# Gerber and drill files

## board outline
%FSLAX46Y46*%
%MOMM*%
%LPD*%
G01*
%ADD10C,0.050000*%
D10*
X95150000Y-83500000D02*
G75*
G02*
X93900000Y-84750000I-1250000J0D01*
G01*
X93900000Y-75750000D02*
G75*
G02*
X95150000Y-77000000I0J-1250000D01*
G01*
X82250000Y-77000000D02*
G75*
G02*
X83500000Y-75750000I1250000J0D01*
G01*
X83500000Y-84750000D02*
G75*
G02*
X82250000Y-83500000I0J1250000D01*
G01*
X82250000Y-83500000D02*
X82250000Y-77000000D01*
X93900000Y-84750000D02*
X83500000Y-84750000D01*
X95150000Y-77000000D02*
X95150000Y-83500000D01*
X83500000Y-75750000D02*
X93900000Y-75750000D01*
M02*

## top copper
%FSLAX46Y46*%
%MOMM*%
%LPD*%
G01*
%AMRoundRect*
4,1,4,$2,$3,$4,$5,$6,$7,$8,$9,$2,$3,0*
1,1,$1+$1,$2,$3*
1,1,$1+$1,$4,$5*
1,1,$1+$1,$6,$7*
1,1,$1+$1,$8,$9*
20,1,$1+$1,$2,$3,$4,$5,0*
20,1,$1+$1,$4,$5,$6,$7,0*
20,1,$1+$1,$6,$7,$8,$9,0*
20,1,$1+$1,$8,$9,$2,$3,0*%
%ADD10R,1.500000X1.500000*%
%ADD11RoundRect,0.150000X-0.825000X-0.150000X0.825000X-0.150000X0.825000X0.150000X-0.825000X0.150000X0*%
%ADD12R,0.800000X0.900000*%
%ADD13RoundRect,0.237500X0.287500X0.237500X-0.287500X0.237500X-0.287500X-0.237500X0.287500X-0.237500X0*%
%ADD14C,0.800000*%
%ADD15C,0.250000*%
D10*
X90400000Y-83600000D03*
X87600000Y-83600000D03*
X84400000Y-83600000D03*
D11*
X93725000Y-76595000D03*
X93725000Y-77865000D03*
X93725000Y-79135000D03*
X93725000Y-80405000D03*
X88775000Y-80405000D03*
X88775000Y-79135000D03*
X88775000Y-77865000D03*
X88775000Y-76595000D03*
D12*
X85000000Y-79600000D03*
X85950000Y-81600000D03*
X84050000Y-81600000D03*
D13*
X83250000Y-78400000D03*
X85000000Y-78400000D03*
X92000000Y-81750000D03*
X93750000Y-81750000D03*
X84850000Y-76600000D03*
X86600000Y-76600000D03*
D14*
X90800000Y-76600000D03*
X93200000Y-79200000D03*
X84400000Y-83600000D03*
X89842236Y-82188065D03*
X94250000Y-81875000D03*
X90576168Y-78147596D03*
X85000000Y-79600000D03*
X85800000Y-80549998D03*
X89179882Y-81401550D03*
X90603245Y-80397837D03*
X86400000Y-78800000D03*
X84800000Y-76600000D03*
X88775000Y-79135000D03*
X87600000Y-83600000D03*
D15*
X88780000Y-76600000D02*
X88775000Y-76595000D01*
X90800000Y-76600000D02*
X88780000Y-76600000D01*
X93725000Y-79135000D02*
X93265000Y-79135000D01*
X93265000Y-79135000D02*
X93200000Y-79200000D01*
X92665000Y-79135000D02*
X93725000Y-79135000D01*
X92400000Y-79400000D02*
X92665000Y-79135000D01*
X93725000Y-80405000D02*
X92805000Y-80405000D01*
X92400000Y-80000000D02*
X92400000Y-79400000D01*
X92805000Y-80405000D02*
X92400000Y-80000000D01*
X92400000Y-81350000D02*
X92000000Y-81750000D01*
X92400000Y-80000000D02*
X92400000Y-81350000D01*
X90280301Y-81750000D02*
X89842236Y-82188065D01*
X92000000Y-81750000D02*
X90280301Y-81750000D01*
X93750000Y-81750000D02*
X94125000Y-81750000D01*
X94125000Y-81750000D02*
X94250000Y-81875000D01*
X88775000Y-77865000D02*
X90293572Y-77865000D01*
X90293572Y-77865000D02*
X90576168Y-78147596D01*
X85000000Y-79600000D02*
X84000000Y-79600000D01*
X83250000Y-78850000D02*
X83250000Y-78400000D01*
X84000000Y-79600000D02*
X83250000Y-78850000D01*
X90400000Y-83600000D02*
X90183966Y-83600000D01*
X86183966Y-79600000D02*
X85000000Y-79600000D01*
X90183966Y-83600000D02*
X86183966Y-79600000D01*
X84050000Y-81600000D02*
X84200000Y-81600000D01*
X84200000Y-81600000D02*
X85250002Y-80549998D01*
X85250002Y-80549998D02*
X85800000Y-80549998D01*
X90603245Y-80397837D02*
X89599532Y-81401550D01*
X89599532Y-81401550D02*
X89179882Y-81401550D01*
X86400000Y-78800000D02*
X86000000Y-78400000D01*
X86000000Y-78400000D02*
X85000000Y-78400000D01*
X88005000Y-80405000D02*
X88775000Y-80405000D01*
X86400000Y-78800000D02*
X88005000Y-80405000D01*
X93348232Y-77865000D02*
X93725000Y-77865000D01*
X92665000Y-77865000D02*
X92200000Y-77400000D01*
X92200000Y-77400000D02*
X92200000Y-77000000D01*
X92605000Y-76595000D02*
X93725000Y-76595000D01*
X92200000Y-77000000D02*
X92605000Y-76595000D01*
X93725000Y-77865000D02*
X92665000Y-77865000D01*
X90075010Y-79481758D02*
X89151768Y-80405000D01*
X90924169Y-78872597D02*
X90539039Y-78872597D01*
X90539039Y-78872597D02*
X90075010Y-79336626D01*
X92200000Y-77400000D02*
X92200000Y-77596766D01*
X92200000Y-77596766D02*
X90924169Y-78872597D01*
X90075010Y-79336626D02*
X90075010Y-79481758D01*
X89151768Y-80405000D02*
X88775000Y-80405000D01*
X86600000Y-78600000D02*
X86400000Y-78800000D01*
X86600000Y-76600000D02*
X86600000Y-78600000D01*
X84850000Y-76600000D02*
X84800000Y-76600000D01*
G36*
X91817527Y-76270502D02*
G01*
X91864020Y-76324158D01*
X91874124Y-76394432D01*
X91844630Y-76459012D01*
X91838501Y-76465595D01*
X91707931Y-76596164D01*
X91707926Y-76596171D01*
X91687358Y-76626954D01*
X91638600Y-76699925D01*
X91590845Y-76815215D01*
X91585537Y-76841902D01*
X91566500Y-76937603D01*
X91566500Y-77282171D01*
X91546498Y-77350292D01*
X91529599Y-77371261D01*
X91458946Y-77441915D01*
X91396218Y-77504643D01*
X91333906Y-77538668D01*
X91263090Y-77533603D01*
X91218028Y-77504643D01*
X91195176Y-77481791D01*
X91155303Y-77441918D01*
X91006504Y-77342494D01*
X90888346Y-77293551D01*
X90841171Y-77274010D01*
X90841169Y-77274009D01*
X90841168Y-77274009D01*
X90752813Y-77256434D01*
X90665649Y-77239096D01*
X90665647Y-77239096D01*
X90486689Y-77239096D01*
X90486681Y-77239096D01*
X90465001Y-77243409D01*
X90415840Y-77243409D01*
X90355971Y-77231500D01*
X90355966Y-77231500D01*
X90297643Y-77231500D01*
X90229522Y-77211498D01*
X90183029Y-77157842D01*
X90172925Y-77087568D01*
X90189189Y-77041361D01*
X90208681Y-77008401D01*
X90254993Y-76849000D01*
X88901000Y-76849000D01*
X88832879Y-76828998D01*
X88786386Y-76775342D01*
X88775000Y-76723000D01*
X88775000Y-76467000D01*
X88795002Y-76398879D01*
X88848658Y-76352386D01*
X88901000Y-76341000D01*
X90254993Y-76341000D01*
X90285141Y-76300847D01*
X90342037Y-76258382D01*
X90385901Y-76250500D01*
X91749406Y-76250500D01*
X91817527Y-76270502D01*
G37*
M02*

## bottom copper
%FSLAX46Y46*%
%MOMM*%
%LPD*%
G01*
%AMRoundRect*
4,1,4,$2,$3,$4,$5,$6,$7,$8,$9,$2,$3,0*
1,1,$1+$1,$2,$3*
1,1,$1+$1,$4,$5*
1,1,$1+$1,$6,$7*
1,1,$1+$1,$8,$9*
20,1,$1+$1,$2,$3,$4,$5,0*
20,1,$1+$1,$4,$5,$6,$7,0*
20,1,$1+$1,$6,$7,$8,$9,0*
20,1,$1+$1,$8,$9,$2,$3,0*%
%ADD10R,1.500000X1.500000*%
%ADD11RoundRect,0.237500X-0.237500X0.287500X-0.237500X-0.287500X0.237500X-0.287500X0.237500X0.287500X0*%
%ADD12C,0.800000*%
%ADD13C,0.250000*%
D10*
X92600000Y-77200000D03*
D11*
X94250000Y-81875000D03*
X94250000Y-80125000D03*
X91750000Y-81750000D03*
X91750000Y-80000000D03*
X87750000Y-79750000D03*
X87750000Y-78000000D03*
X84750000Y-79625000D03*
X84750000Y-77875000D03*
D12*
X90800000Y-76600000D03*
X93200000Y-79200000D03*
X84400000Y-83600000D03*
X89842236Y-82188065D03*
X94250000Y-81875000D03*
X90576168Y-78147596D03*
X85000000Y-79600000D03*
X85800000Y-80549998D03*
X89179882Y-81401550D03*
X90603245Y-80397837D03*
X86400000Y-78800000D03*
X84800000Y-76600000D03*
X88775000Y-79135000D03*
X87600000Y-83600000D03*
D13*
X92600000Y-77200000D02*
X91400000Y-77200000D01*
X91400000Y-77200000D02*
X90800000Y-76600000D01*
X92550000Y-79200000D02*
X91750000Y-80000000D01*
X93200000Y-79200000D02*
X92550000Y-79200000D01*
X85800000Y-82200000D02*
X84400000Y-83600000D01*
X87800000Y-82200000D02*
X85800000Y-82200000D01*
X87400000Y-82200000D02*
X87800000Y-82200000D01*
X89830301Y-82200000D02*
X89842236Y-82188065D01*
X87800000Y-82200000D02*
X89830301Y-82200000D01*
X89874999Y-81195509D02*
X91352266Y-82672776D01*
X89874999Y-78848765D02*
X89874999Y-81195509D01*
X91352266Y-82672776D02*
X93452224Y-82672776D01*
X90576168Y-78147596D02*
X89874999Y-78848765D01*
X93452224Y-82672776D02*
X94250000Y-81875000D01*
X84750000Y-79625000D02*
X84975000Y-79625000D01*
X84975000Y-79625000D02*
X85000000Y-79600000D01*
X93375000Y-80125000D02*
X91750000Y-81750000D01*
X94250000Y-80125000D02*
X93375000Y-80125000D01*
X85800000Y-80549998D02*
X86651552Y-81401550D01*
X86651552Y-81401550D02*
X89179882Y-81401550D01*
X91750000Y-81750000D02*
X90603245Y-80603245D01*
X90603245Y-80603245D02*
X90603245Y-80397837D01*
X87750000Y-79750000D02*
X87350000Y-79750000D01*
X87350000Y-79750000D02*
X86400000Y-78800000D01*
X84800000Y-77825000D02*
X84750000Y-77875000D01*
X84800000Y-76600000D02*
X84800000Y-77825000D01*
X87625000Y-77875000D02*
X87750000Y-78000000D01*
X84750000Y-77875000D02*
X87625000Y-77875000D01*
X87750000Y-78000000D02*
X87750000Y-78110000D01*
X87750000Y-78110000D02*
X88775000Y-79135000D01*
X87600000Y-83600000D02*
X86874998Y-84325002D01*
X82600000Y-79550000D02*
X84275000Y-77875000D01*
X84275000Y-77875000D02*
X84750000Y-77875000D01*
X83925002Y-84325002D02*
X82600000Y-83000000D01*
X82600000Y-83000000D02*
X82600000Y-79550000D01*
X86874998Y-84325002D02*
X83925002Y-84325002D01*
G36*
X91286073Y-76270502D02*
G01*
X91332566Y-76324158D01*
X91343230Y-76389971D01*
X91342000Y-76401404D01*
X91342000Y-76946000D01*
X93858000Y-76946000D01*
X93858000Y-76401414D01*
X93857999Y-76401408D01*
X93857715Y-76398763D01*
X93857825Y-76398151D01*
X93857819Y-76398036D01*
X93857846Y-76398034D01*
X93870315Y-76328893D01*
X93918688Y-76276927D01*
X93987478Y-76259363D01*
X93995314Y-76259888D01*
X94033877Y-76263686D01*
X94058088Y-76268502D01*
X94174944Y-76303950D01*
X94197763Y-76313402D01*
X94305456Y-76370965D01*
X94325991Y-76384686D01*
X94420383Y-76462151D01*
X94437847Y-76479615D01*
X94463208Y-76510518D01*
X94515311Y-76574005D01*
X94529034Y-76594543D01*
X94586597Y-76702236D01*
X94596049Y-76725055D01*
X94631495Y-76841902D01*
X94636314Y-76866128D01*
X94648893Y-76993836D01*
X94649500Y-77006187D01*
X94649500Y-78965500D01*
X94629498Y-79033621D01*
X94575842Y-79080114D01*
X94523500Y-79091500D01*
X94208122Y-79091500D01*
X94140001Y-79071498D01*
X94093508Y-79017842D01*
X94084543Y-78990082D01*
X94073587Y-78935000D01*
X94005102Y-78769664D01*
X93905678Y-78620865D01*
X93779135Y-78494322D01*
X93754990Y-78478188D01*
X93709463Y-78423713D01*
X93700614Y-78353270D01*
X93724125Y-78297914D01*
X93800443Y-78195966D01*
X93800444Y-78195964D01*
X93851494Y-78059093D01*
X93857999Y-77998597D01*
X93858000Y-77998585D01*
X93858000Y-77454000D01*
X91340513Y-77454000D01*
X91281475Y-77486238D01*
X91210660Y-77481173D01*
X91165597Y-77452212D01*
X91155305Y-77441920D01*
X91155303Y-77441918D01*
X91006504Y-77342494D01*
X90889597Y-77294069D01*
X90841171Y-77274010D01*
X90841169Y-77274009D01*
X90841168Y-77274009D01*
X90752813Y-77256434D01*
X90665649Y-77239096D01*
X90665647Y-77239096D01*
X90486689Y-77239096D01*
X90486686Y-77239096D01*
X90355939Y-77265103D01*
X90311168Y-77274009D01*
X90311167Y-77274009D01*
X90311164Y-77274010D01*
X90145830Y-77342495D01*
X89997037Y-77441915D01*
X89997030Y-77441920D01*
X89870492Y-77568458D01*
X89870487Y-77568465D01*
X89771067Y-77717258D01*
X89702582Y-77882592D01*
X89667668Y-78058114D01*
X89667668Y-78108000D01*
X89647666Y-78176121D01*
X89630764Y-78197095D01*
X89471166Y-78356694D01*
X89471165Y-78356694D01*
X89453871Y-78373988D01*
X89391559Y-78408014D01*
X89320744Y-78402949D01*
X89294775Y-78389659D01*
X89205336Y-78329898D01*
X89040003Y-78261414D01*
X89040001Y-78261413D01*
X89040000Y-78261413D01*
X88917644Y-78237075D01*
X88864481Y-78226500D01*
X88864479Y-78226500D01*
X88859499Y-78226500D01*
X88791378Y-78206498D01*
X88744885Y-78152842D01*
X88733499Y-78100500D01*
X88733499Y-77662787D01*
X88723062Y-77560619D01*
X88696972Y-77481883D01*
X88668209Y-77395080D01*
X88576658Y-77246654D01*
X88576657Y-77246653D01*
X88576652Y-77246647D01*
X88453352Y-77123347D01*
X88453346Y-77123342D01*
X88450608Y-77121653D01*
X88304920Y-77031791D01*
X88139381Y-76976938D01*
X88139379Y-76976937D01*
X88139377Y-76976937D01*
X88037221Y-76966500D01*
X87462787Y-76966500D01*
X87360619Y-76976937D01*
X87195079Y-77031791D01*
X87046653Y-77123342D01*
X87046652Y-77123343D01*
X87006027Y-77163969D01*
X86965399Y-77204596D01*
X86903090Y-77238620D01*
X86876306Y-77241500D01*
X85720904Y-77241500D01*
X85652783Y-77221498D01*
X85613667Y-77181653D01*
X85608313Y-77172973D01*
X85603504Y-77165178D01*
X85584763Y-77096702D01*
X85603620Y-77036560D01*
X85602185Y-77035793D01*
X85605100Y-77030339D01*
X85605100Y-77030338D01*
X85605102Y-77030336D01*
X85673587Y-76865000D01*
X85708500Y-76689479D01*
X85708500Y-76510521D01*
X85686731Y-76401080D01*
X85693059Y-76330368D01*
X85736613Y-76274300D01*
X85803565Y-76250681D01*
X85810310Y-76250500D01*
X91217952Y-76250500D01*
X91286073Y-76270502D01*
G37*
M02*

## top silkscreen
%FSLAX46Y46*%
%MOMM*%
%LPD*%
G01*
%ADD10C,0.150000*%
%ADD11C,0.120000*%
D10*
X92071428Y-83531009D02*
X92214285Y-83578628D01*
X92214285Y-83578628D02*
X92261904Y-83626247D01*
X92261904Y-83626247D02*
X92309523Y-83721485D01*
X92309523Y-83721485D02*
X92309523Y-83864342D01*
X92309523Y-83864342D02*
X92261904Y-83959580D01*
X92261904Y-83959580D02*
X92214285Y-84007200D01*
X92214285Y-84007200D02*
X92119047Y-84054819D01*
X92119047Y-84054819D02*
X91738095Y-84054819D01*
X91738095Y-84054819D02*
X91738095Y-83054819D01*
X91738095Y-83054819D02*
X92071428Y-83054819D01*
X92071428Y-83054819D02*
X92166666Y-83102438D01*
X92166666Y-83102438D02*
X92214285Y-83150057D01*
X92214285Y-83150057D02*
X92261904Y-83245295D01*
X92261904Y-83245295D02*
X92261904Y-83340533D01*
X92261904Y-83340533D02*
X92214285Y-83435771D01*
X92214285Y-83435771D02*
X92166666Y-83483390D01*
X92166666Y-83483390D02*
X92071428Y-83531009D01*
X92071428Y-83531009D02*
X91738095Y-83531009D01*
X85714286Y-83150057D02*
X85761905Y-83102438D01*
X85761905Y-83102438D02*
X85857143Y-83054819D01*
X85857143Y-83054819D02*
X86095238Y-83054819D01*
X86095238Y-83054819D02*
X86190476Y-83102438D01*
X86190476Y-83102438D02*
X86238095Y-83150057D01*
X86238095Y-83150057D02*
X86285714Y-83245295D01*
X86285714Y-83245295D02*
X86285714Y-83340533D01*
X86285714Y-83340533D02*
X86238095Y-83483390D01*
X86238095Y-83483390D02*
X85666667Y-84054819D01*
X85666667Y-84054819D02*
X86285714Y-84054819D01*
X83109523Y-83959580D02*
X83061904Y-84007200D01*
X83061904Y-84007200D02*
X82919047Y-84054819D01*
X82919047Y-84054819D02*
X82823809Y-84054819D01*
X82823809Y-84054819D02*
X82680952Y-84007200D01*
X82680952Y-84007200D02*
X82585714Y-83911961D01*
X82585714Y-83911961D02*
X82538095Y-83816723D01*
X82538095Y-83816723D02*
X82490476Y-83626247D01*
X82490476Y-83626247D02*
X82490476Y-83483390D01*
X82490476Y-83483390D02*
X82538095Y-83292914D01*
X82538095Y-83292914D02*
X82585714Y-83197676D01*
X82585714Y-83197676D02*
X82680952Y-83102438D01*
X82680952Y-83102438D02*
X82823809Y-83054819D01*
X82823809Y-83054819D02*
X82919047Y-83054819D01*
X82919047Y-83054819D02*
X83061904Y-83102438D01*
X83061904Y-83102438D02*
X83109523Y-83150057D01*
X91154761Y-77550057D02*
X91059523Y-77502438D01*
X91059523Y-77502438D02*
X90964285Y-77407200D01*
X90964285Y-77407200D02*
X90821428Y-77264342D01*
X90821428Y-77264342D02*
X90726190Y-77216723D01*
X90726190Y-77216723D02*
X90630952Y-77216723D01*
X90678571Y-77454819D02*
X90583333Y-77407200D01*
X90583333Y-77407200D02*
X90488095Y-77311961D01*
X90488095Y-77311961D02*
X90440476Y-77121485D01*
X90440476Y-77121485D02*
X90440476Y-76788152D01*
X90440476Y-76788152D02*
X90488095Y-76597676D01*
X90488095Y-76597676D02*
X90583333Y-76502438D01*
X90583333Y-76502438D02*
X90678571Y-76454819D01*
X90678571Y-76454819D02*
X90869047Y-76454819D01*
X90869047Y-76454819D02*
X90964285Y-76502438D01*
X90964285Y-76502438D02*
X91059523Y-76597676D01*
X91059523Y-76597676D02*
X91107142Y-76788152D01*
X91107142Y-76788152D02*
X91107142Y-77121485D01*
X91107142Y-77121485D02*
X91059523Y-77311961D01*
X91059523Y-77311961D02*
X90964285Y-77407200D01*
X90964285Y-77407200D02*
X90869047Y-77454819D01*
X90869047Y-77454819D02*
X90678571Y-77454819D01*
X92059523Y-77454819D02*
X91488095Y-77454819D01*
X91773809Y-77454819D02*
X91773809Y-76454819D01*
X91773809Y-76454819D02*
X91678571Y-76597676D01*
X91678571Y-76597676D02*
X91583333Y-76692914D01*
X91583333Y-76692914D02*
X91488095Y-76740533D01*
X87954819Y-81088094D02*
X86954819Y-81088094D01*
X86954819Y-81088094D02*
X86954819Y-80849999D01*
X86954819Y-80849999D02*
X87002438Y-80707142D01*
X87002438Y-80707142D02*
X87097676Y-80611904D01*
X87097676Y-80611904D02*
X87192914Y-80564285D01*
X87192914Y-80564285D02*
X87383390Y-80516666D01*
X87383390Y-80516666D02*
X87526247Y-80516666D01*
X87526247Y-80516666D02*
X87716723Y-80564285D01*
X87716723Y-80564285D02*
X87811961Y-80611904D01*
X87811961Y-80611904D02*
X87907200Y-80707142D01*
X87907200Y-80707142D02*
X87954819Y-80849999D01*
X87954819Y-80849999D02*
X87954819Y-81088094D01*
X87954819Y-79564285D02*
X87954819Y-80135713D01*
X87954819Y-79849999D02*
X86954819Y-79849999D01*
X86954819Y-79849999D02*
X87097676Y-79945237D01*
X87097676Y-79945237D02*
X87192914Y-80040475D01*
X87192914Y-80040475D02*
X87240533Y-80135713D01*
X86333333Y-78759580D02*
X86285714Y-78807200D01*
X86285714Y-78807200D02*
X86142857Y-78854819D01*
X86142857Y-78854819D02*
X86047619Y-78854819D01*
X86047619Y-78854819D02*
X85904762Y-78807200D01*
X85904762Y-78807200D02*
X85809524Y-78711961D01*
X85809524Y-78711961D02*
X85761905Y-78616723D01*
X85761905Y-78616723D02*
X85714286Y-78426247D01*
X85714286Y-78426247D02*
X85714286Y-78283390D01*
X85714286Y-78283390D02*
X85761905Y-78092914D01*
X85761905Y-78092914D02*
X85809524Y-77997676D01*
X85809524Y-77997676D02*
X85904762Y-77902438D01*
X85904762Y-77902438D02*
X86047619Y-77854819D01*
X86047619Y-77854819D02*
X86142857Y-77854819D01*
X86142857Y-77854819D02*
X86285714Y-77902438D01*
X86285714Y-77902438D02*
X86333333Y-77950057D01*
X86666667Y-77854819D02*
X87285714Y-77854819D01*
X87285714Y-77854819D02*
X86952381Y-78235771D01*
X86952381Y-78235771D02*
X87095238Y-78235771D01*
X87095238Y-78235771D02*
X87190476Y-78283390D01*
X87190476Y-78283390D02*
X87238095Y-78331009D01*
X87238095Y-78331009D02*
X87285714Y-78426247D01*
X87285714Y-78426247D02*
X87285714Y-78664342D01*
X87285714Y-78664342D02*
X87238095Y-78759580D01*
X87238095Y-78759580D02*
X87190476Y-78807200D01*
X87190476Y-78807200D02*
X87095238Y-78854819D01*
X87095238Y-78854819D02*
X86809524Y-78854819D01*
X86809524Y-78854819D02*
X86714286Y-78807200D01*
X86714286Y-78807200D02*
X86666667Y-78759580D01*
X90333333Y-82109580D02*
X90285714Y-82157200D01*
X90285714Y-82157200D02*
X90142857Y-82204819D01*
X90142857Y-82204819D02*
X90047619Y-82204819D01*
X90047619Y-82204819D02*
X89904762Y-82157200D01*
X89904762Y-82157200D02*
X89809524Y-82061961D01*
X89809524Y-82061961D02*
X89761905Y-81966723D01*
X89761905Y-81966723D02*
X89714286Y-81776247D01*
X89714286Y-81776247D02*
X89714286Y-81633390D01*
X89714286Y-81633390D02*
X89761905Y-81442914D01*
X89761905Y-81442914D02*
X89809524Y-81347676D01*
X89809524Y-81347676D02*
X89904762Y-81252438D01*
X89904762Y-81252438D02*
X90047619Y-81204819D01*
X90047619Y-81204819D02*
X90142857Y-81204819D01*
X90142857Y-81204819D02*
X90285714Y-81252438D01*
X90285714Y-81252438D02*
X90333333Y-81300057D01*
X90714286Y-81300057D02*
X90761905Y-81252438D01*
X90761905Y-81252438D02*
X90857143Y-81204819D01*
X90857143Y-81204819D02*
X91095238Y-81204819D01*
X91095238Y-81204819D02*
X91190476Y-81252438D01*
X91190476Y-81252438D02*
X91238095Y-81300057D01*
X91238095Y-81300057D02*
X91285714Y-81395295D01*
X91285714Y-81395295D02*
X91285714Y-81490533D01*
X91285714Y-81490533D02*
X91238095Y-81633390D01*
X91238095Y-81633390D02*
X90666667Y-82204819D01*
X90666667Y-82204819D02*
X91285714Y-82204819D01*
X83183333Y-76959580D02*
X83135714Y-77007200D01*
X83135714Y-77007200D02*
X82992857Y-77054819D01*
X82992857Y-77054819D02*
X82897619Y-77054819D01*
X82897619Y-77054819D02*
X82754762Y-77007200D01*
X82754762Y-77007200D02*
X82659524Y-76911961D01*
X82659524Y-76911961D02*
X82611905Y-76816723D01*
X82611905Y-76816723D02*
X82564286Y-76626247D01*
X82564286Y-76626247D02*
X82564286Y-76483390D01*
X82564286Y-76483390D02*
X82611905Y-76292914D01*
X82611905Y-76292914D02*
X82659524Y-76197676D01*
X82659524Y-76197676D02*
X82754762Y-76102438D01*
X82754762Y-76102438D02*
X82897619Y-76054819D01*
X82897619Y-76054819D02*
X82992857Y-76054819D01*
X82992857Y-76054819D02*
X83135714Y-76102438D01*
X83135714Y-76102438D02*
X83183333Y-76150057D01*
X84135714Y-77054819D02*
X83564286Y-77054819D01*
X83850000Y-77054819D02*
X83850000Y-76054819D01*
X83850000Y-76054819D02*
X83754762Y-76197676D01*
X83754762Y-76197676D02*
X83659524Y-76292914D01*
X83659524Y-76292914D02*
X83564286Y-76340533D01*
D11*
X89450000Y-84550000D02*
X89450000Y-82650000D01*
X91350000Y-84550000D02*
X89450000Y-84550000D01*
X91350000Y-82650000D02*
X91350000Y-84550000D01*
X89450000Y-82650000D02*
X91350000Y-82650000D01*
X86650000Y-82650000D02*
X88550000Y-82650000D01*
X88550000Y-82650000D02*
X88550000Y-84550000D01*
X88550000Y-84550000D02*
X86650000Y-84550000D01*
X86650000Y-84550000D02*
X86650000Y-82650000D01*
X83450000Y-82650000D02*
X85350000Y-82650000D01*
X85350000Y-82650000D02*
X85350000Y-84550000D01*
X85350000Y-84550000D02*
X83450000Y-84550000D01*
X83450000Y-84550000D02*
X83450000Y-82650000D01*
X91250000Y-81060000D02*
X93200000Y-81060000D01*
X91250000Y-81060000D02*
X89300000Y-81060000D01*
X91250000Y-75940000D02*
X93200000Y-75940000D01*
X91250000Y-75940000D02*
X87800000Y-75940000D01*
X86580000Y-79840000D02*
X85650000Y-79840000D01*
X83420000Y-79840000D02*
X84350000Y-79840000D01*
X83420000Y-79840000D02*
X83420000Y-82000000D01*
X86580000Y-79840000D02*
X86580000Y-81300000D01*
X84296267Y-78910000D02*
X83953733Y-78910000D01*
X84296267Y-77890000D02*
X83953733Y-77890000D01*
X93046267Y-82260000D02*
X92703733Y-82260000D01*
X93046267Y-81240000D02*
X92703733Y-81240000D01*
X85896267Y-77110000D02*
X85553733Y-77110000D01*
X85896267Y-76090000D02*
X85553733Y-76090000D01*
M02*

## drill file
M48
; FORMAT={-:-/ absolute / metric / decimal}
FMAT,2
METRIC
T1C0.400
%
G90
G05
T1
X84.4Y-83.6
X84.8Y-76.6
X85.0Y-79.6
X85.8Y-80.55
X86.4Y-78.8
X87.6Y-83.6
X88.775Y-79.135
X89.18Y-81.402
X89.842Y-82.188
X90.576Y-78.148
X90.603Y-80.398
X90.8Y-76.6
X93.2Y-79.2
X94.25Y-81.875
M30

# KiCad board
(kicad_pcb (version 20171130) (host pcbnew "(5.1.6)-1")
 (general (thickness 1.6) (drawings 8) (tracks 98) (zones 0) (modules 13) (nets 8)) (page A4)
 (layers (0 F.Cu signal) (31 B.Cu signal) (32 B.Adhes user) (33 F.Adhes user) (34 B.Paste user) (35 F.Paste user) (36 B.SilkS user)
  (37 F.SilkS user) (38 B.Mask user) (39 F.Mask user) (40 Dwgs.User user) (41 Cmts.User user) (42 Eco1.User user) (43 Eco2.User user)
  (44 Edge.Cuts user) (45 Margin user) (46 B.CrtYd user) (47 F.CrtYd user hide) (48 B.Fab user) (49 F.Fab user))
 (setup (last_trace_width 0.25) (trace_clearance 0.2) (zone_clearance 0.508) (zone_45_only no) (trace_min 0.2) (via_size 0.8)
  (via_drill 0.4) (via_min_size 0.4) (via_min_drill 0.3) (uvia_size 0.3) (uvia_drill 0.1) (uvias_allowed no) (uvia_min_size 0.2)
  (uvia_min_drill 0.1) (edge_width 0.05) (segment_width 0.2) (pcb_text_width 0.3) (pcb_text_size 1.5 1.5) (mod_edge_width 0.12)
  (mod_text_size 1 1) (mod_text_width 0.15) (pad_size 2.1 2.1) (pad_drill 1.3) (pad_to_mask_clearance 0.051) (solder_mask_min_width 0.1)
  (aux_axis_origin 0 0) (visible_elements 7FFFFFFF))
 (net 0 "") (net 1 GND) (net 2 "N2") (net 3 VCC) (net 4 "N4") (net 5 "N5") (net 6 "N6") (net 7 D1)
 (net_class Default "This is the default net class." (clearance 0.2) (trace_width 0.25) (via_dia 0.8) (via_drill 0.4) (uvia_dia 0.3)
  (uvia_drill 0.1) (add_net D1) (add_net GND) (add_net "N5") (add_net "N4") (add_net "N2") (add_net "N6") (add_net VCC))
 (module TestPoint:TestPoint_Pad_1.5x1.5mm (layer B.Cu) (at 92.6 77.2 90)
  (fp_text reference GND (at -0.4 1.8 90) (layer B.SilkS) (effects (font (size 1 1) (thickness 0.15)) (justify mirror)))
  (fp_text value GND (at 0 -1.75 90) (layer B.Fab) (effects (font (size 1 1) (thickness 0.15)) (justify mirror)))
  (pad 1 smd rect (at 0 0 90) (size 1.5 1.5) (layers B.Cu B.Mask) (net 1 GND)))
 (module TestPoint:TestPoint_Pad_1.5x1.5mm (layer F.Cu) (at 90.4 83.6)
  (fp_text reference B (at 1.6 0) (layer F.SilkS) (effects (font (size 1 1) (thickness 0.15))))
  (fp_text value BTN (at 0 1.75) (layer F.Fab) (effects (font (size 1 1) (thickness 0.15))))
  (fp_line (start -0.95 0.95) (end -0.95 -0.95) (layer F.SilkS) (width 0.12))
  (fp_line (start 0.95 0.95) (end -0.95 0.95) (layer F.SilkS) (width 0.12))
  (fp_line (start 0.95 -0.95) (end 0.95 0.95) (layer F.SilkS) (width 0.12))
  (fp_line (start -0.95 -0.95) (end 0.95 -0.95) (layer F.SilkS) (width 0.12))
  (pad 1 smd rect (at 0 0) (size 1.5 1.5) (layers F.Cu F.Mask) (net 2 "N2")))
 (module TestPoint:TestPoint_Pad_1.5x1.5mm (layer F.Cu) (at 87.6 83.6)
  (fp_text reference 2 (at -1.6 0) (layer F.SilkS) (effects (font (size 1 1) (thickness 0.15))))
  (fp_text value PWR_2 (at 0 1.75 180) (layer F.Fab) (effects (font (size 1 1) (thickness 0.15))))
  (fp_line (start -0.95 -0.95) (end 0.95 -0.95) (layer F.SilkS) (width 0.12))
  (fp_line (start 0.95 -0.95) (end 0.95 0.95) (layer F.SilkS) (width 0.12))
  (fp_line (start 0.95 0.95) (end -0.95 0.95) (layer F.SilkS) (width 0.12))
  (fp_line (start -0.95 0.95) (end -0.95 -0.95) (layer F.SilkS) (width 0.12))
  (pad 1 smd rect (at 0 0) (size 1.5 1.5) (layers F.Cu F.Mask) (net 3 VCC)))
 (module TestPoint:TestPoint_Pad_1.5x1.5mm (layer F.Cu) (at 84.4 83.6)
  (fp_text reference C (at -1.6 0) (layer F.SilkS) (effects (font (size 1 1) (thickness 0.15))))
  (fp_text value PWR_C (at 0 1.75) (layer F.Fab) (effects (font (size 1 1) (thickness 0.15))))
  (fp_line (start -0.95 -0.95) (end 0.95 -0.95) (layer F.SilkS) (width 0.12))
  (fp_line (start 0.95 -0.95) (end 0.95 0.95) (layer F.SilkS) (width 0.12))
  (fp_line (start 0.95 0.95) (end -0.95 0.95) (layer F.SilkS) (width 0.12))
  (fp_line (start -0.95 0.95) (end -0.95 -0.95) (layer F.SilkS) (width 0.12))
  (pad 1 smd rect (at 0 0) (size 1.5 1.5) (layers F.Cu F.Mask) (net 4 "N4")))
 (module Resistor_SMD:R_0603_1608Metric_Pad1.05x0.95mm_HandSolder (layer B.Cu) (at 94.25 81 270)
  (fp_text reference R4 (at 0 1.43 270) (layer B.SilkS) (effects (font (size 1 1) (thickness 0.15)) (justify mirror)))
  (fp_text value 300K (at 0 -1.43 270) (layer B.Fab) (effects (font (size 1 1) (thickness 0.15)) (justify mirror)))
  (pad 2 smd roundrect (at 0.875 0 270) (size 1.05 0.95) (layers B.Cu B.Paste B.Mask) (roundrect_rratio 0.25) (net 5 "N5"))
  (pad 1 smd roundrect (at -0.875 0 270) (size 1.05 0.95) (layers B.Cu B.Paste B.Mask) (roundrect_rratio 0.25) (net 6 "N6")))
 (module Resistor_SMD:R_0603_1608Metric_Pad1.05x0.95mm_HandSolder (layer B.Cu) (at 91.75 80.875 270)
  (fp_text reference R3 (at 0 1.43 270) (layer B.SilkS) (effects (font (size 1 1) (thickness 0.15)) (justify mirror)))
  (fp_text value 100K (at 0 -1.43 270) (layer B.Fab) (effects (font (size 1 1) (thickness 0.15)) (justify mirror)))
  (pad 2 smd roundrect (at 0.875 0 270) (size 1.05 0.95) (layers B.Cu B.Paste B.Mask) (roundrect_rratio 0.25) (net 6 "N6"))
  (pad 1 smd roundrect (at -0.875 0 270) (size 1.05 0.95) (layers B.Cu B.Paste B.Mask) (roundrect_rratio 0.25) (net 4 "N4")))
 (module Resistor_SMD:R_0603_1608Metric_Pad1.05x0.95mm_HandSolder (layer B.Cu) (at 87.75 78.875 270)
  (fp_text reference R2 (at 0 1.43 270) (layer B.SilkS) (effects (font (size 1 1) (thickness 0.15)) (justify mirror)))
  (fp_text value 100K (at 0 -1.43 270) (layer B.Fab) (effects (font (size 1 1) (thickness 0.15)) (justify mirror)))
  (pad 2 smd roundrect (at 0.875 0 270) (size 1.05 0.95) (layers B.Cu B.Paste B.Mask) (roundrect_rratio 0.25) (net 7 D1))
  (pad 1 smd roundrect (at -0.875 0 270) (size 1.05 0.95) (layers B.Cu B.Paste B.Mask) (roundrect_rratio 0.25) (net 3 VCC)))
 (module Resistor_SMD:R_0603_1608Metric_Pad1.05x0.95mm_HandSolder (layer B.Cu) (at 84.75 78.75 270)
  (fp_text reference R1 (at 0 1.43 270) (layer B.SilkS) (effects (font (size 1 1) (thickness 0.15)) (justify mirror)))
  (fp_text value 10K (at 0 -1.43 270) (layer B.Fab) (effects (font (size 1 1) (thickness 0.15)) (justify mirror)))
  (pad 2 smd roundrect (at 0.875 0 270) (size 1.05 0.95) (layers B.Cu B.Paste B.Mask) (roundrect_rratio 0.25) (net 2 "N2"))
  (pad 1 smd roundrect (at -0.875 0 270) (size 1.05 0.95) (layers B.Cu B.Paste B.Mask) (roundrect_rratio 0.25) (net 3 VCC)))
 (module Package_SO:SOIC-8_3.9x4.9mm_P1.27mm (layer F.Cu) (at 91.25 78.5)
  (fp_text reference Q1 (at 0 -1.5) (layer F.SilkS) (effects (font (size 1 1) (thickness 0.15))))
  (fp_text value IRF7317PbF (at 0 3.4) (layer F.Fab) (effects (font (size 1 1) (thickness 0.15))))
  (fp_line (start 0 2.56) (end 1.95 2.56) (layer F.SilkS) (width 0.12))
  (fp_line (start 0 2.56) (end -1.95 2.56) (layer F.SilkS) (width 0.12))
  (fp_line (start 0 -2.56) (end 1.95 -2.56) (layer F.SilkS) (width 0.12))
  (fp_line (start 0 -2.56) (end -3.45 -2.56) (layer F.SilkS) (width 0.12))
  (pad 8 smd roundrect (at 2.475 -1.905) (size 1.95 0.6) (layers F.Cu F.Paste F.Mask) (roundrect_rratio 0.25) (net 7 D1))
  (pad 7 smd roundrect (at 2.475 -0.635) (size 1.95 0.6) (layers F.Cu F.Paste F.Mask) (roundrect_rratio 0.25) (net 7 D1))
  (pad 6 smd roundrect (at 2.475 0.635) (size 1.95 0.6) (layers F.Cu F.Paste F.Mask) (roundrect_rratio 0.25) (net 4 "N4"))
  (pad 5 smd roundrect (at 2.475 1.905) (size 1.95 0.6) (layers F.Cu F.Paste F.Mask) (roundrect_rratio 0.25) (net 4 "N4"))
  (pad 4 smd roundrect (at -2.475 1.905) (size 1.95 0.6) (layers F.Cu F.Paste F.Mask) (roundrect_rratio 0.25) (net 7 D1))
  (pad 3 smd roundrect (at -2.475 0.635) (size 1.95 0.6) (layers F.Cu F.Paste F.Mask) (roundrect_rratio 0.25) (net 3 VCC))
  (pad 2 smd roundrect (at -2.475 -0.635) (size 1.95 0.6) (layers F.Cu F.Paste F.Mask) (roundrect_rratio 0.25) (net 5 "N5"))
  (pad 1 smd roundrect (at -2.475 -1.905) (size 1.95 0.6) (layers F.Cu F.Paste F.Mask) (roundrect_rratio 0.25) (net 1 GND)))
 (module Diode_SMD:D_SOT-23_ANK (layer F.Cu) (at 85 80.6 90)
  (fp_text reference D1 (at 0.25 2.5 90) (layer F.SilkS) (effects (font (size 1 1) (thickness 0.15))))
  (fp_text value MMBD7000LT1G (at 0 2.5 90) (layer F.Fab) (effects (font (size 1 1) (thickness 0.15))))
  (fp_line (start 0.76 1.58) (end 0.76 0.65) (layer F.SilkS) (width 0.12))
  (fp_line (start 0.76 -1.58) (end 0.76 -0.65) (layer F.SilkS) (width 0.12))
  (fp_line (start 0.76 -1.58) (end -1.4 -1.58) (layer F.SilkS) (width 0.12))
  (fp_line (start 0.76 1.58) (end -0.7 1.58) (layer F.SilkS) (width 0.12))
  (pad 1 smd rect (at 1 0 90) (size 0.9 0.8) (layers F.Cu F.Paste F.Mask) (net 2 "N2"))
  (pad "" smd rect (at -1 0.95 90) (size 0.9 0.8) (layers F.Cu F.Paste F.Mask))
  (pad 2 smd rect (at -1 -0.95 90) (size 0.9 0.8) (layers F.Cu F.Paste F.Mask) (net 6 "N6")))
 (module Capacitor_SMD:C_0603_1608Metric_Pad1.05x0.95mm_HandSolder (layer F.Cu) (at 84.125 78.4 180)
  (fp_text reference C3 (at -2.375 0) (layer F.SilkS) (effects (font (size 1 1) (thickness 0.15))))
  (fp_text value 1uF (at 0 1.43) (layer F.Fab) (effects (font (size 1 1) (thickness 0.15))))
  (fp_line (start -0.171267 -0.51) (end 0.171267 -0.51) (layer F.SilkS) (width 0.12))
  (fp_line (start -0.171267 0.51) (end 0.171267 0.51) (layer F.SilkS) (width 0.12))
  (pad 2 smd roundrect (at 0.875 0 180) (size 1.05 0.95) (layers F.Cu F.Paste F.Mask) (roundrect_rratio 0.25) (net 2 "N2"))
  (pad 1 smd roundrect (at -0.875 0 180) (size 1.05 0.95) (layers F.Cu F.Paste F.Mask) (roundrect_rratio 0.25) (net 7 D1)))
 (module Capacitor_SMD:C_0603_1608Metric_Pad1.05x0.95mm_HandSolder (layer F.Cu) (at 92.875 81.75 180)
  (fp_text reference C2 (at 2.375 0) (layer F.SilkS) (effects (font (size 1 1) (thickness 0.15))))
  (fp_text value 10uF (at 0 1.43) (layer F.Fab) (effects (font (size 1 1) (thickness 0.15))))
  (fp_line (start -0.171267 -0.51) (end 0.171267 -0.51) (layer F.SilkS) (width 0.12))
  (fp_line (start -0.171267 0.51) (end 0.171267 0.51) (layer F.SilkS) (width 0.12))
  (pad 2 smd roundrect (at 0.875 0 180) (size 1.05 0.95) (layers F.Cu F.Paste F.Mask) (roundrect_rratio 0.25) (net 4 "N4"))
  (pad 1 smd roundrect (at -0.875 0 180) (size 1.05 0.95) (layers F.Cu F.Paste F.Mask) (roundrect_rratio 0.25) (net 5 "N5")))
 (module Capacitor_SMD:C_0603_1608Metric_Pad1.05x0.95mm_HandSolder (layer F.Cu) (at 85.725 76.6 180)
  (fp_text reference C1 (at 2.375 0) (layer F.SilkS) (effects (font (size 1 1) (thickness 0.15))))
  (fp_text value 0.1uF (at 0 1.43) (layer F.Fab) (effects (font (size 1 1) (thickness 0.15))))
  (fp_line (start -0.171267 -0.51) (end 0.171267 -0.51) (layer F.SilkS) (width 0.12))
  (fp_line (start -0.171267 0.51) (end 0.171267 0.51) (layer F.SilkS) (width 0.12))
  (pad 2 smd roundrect (at 0.875 0 180) (size 1.05 0.95) (layers F.Cu F.Paste F.Mask) (roundrect_rratio 0.25) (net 3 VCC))
  (pad 1 smd roundrect (at -0.875 0 180) (size 1.05 0.95) (layers F.Cu F.Paste F.Mask) (roundrect_rratio 0.25) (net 7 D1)))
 (gr_arc (start 93.9 83.5) (end 93.9 84.75) (angle -90) (layer Edge.Cuts) (width 0.05))
 (gr_arc (start 93.9 77) (end 95.15 77) (angle -90) (layer Edge.Cuts) (width 0.05))
 (gr_arc (start 83.5 77) (end 83.5 75.75) (angle -90) (layer Edge.Cuts) (width 0.05))
 (gr_arc (start 83.5 83.5) (end 82.25 83.5) (angle -90) (layer Edge.Cuts) (width 0.05))
 (gr_line (start 82.25 83.5) (end 82.25 77) (layer Edge.Cuts) (width 0.05))
 (gr_line (start 93.9 84.75) (end 83.5 84.75) (layer Edge.Cuts) (width 0.05))
 (gr_line (start 95.15 77) (end 95.15 83.5) (layer Edge.Cuts) (width 0.05))
 (gr_line (start 83.5 75.75) (end 93.9 75.75) (layer Edge.Cuts) (width 0.05))
 (segment (start 92.6 77.2) (end 91.4 77.2) (width 0.25) (layer B.Cu) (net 1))
 (via (at 90.8 76.6) (size 0.8) (drill 0.4) (layers F.Cu B.Cu) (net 1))
 (segment (start 91.4 77.2) (end 90.8 76.6) (width 0.25) (layer B.Cu) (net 1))
 (segment (start 88.78 76.6) (end 88.775 76.595) (width 0.25) (layer F.Cu) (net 1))
 (segment (start 90.8 76.6) (end 88.78 76.6) (width 0.25) (layer F.Cu) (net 1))
 (via (at 93.2 79.2) (size 0.8) (drill 0.4) (layers F.Cu B.Cu) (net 4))
 (segment (start 93.725 79.135) (end 93.265 79.135) (width 0.25) (layer F.Cu) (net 4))
 (segment (start 93.265 79.135) (end 93.2 79.2) (width 0.25) (layer F.Cu) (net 4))
 (segment (start 92.55 79.2) (end 91.75 80) (width 0.25) (layer B.Cu) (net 4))
 (segment (start 93.2 79.2) (end 92.55 79.2) (width 0.25) (layer B.Cu) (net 4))
 (segment (start 92.665 79.135) (end 93.725 79.135) (width 0.25) (layer F.Cu) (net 4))
 (segment (start 92.4 79.4) (end 92.665 79.135) (width 0.25) (layer F.Cu) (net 4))
 (segment (start 93.725 80.405) (end 92.805 80.405) (width 0.25) (layer F.Cu) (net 4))
 (segment (start 92.4 80) (end 92.4 79.4) (width 0.25) (layer F.Cu) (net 4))
 (segment (start 92.805 80.405) (end 92.4 80) (width 0.25) (layer F.Cu) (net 4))
 (segment (start 92.4 81.35) (end 92 81.75) (width 0.25) (layer F.Cu) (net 4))
 (segment (start 92.4 80) (end 92.4 81.35) (width 0.25) (layer F.Cu) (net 4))
 (via (at 84.4 83.6) (size 0.8) (drill 0.4) (layers F.Cu B.Cu) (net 4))
 (segment (start 85.8 82.2) (end 84.4 83.6) (width 0.25) (layer B.Cu) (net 4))
 (segment (start 87.8 82.2) (end 85.8 82.2) (width 0.25) (layer B.Cu) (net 4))
 (segment (start 87.4 82.2) (end 87.8 82.2) (width 0.25) (layer B.Cu) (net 4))
 (segment (start 89.830301 82.2) (end 89.842236 82.188065) (width 0.25) (layer B.Cu) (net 4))
 (segment (start 90.280301 81.75) (end 89.842236 82.188065) (width 0.25) (layer F.Cu) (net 4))
 (segment (start 87.8 82.2) (end 89.830301 82.2) (width 0.25) (layer B.Cu) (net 4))
 (segment (start 92 81.75) (end 90.280301 81.75) (width 0.25) (layer F.Cu) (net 4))
 (via (at 89.842236 82.188065) (size 0.8) (drill 0.4) (layers F.Cu B.Cu) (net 4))
 (via (at 94.25 81.875) (size 0.8) (drill 0.4) (layers F.Cu B.Cu) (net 5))
 (segment (start 93.75 81.75) (end 94.125 81.75) (width 0.25) (layer F.Cu) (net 5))
 (segment (start 94.125 81.75) (end 94.25 81.875) (width 0.25) (layer F.Cu) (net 5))
 (segment (start 88.775 77.865) (end 90.293572 77.865) (width 0.25) (layer F.Cu) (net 5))
 (segment (start 90.293572 77.865) (end 90.576168 78.147596) (width 0.25) (layer F.Cu) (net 5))
 (via (at 90.576168 78.147596) (size 0.8) (drill 0.4) (layers F.Cu B.Cu) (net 5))
 (segment (start 89.874999 81.195509) (end 91.352266 82.672776) (width 0.25) (layer B.Cu) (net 5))
 (segment (start 89.874999 78.848765) (end 89.874999 81.195509) (width 0.25) (layer B.Cu) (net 5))
 (segment (start 91.352266 82.672776) (end 93.452224 82.672776) (width 0.25) (layer B.Cu) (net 5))
 (segment (start 90.576168 78.147596) (end 89.874999 78.848765) (width 0.25) (layer B.Cu) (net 5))
 (segment (start 93.452224 82.672776) (end 94.25 81.875) (width 0.25) (layer B.Cu) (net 5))
 (segment (start 85 79.6) (end 84 79.6) (width 0.25) (layer F.Cu) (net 2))
 (segment (start 83.25 78.85) (end 83.25 78.4) (width 0.25) (layer F.Cu) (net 2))
 (segment (start 84 79.6) (end 83.25 78.85) (width 0.25) (layer F.Cu) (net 2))
 (segment (start 84.75 79.625) (end 84.975 79.625) (width 0.25) (layer B.Cu) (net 2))
 (via (at 85 79.6) (size 0.8) (drill 0.4) (layers F.Cu B.Cu) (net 2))
 (segment (start 84.975 79.625) (end 85 79.6) (width 0.25) (layer B.Cu) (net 2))
 (segment (start 90.4 83.6) (end 90.183966 83.6) (width 0.25) (layer F.Cu) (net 2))
 (segment (start 86.183966 79.6) (end 85 79.6) (width 0.25) (layer F.Cu) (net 2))
 (segment (start 90.183966 83.6) (end 86.183966 79.6) (width 0.25) (layer F.Cu) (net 2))
 (segment (start 93.375 80.125) (end 91.75 81.75) (width 0.25) (layer B.Cu) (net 6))
 (segment (start 94.25 80.125) (end 93.375 80.125) (width 0.25) (layer B.Cu) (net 6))
 (segment (start 84.05 81.6) (end 84.2 81.6) (width 0.25) (layer F.Cu) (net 6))
 (via (at 85.8 80.549998) (size 0.8) (drill 0.4) (layers F.Cu B.Cu) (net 6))
 (segment (start 84.2 81.6) (end 85.250002 80.549998) (width 0.25) (layer F.Cu) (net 6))
 (segment (start 85.250002 80.549998) (end 85.8 80.549998) (width 0.25) (layer F.Cu) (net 6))
 (via (at 89.179882 81.40155) (size 0.8) (drill 0.4) (layers F.Cu B.Cu) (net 6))
 (via (at 90.603245 80.397837) (size 0.8) (drill 0.4) (layers F.Cu B.Cu) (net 6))
 (segment (start 90.603245 80.397837) (end 89.599532 81.40155) (width 0.25) (layer F.Cu) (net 6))
 (segment (start 85.8 80.549998) (end 86.651552 81.40155) (width 0.25) (layer B.Cu) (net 6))
 (segment (start 89.599532 81.40155) (end 89.179882 81.40155) (width 0.25) (layer F.Cu) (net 6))
 (segment (start 86.651552 81.40155) (end 89.179882 81.40155) (width 0.25) (layer B.Cu) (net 6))
 (segment (start 91.75 81.75) (end 90.603245 80.603245) (width 0.25) (layer B.Cu) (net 6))
 (segment (start 90.603245 80.603245) (end 90.603245 80.397837) (width 0.25) (layer B.Cu) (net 6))
 (via (at 86.4 78.8) (size 0.8) (drill 0.4) (layers F.Cu B.Cu) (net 7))
 (segment (start 87.75 79.75) (end 87.35 79.75) (width 0.25) (layer B.Cu) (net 7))
 (segment (start 87.35 79.75) (end 86.4 78.8) (width 0.25) (layer B.Cu) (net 7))
 (segment (start 86.4 78.8) (end 86 78.4) (width 0.25) (layer F.Cu) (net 7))
 (segment (start 86 78.4) (end 85 78.4) (width 0.25) (layer F.Cu) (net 7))
 (segment (start 88.005 80.405) (end 88.775 80.405) (width 0.25) (layer F.Cu) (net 7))
 (segment (start 86.4 78.8) (end 88.005 80.405) (width 0.25) (layer F.Cu) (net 7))
 (segment (start 93.348232 77.865) (end 93.725 77.865) (width 0.25) (layer F.Cu) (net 7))
 (segment (start 92.665 77.865) (end 92.2 77.4) (width 0.25) (layer F.Cu) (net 7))
 (segment (start 92.2 77.4) (end 92.2 77) (width 0.25) (layer F.Cu) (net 7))
 (segment (start 92.605 76.595) (end 93.725 76.595) (width 0.25) (layer F.Cu) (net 7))
 (segment (start 92.2 77) (end 92.605 76.595) (width 0.25) (layer F.Cu) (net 7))
 (segment (start 93.725 77.865) (end 92.665 77.865) (width 0.25) (layer F.Cu) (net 7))
 (segment (start 90.07501 79.481758) (end 89.151768 80.405) (width 0.25) (layer F.Cu) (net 7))
 (segment (start 90.924169 78.872597) (end 90.539039 78.872597) (width 0.25) (layer F.Cu) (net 7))
 (segment (start 90.539039 78.872597) (end 90.07501 79.336626) (width 0.25) (layer F.Cu) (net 7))
 (segment (start 92.2 77.4) (end 92.2 77.596766) (width 0.25) (layer F.Cu) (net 7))
 (segment (start 92.2 77.596766) (end 90.924169 78.872597) (width 0.25) (layer F.Cu) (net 7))
 (segment (start 90.07501 79.336626) (end 90.07501 79.481758) (width 0.25) (layer F.Cu) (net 7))
 (segment (start 89.151768 80.405) (end 88.775 80.405) (width 0.25) (layer F.Cu) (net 7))
 (segment (start 86.6 78.6) (end 86.4 78.8) (width 0.25) (layer F.Cu) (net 7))
 (segment (start 86.6 76.6) (end 86.6 78.6) (width 0.25) (layer F.Cu) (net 7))
 (via (at 84.8 76.6) (size 0.8) (drill 0.4) (layers F.Cu B.Cu) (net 3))
 (segment (start 84.85 76.6) (end 84.8 76.6) (width 0.25) (layer F.Cu) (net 3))
 (segment (start 84.8 77.825) (end 84.75 77.875) (width 0.25) (layer B.Cu) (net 3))
 (segment (start 84.8 76.6) (end 84.8 77.825) (width 0.25) (layer B.Cu) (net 3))
 (segment (start 87.625 77.875) (end 87.75 78) (width 0.25) (layer B.Cu) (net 3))
 (segment (start 84.75 77.875) (end 87.625 77.875) (width 0.25) (layer B.Cu) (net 3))
 (via (at 88.775 79.135) (size 0.8) (drill 0.4) (layers F.Cu B.Cu) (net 3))
 (segment (start 87.75 78) (end 87.75 78.11) (width 0.25) (layer B.Cu) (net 3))
 (segment (start 87.75 78.11) (end 88.775 79.135) (width 0.25) (layer B.Cu) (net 3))
 (via (at 87.6 83.6) (size 0.8) (drill 0.4) (layers F.Cu B.Cu) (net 3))
 (segment (start 87.6 83.6) (end 86.874998 84.325002) (width 0.25) (layer B.Cu) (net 3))
 (segment (start 82.6 79.55) (end 84.275 77.875) (width 0.25) (layer B.Cu) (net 3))
 (segment (start 84.275 77.875) (end 84.75 77.875) (width 0.25) (layer B.Cu) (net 3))
 (segment (start 83.925002 84.325002) (end 82.6 83) (width 0.25) (layer B.Cu) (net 3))
 (segment (start 82.6 83) (end 82.6 79.55) (width 0.25) (layer B.Cu) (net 3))
 (segment (start 86.874998 84.325002) (end 83.925002 84.325002) (width 0.25) (layer B.Cu) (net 3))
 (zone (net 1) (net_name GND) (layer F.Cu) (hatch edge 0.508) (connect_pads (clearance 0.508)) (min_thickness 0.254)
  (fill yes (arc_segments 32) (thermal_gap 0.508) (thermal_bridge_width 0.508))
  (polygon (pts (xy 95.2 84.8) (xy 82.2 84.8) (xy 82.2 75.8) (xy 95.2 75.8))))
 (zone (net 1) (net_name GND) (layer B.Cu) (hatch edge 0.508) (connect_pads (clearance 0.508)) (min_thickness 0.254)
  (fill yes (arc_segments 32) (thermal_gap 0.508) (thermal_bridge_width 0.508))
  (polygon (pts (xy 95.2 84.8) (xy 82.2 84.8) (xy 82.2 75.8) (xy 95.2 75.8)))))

